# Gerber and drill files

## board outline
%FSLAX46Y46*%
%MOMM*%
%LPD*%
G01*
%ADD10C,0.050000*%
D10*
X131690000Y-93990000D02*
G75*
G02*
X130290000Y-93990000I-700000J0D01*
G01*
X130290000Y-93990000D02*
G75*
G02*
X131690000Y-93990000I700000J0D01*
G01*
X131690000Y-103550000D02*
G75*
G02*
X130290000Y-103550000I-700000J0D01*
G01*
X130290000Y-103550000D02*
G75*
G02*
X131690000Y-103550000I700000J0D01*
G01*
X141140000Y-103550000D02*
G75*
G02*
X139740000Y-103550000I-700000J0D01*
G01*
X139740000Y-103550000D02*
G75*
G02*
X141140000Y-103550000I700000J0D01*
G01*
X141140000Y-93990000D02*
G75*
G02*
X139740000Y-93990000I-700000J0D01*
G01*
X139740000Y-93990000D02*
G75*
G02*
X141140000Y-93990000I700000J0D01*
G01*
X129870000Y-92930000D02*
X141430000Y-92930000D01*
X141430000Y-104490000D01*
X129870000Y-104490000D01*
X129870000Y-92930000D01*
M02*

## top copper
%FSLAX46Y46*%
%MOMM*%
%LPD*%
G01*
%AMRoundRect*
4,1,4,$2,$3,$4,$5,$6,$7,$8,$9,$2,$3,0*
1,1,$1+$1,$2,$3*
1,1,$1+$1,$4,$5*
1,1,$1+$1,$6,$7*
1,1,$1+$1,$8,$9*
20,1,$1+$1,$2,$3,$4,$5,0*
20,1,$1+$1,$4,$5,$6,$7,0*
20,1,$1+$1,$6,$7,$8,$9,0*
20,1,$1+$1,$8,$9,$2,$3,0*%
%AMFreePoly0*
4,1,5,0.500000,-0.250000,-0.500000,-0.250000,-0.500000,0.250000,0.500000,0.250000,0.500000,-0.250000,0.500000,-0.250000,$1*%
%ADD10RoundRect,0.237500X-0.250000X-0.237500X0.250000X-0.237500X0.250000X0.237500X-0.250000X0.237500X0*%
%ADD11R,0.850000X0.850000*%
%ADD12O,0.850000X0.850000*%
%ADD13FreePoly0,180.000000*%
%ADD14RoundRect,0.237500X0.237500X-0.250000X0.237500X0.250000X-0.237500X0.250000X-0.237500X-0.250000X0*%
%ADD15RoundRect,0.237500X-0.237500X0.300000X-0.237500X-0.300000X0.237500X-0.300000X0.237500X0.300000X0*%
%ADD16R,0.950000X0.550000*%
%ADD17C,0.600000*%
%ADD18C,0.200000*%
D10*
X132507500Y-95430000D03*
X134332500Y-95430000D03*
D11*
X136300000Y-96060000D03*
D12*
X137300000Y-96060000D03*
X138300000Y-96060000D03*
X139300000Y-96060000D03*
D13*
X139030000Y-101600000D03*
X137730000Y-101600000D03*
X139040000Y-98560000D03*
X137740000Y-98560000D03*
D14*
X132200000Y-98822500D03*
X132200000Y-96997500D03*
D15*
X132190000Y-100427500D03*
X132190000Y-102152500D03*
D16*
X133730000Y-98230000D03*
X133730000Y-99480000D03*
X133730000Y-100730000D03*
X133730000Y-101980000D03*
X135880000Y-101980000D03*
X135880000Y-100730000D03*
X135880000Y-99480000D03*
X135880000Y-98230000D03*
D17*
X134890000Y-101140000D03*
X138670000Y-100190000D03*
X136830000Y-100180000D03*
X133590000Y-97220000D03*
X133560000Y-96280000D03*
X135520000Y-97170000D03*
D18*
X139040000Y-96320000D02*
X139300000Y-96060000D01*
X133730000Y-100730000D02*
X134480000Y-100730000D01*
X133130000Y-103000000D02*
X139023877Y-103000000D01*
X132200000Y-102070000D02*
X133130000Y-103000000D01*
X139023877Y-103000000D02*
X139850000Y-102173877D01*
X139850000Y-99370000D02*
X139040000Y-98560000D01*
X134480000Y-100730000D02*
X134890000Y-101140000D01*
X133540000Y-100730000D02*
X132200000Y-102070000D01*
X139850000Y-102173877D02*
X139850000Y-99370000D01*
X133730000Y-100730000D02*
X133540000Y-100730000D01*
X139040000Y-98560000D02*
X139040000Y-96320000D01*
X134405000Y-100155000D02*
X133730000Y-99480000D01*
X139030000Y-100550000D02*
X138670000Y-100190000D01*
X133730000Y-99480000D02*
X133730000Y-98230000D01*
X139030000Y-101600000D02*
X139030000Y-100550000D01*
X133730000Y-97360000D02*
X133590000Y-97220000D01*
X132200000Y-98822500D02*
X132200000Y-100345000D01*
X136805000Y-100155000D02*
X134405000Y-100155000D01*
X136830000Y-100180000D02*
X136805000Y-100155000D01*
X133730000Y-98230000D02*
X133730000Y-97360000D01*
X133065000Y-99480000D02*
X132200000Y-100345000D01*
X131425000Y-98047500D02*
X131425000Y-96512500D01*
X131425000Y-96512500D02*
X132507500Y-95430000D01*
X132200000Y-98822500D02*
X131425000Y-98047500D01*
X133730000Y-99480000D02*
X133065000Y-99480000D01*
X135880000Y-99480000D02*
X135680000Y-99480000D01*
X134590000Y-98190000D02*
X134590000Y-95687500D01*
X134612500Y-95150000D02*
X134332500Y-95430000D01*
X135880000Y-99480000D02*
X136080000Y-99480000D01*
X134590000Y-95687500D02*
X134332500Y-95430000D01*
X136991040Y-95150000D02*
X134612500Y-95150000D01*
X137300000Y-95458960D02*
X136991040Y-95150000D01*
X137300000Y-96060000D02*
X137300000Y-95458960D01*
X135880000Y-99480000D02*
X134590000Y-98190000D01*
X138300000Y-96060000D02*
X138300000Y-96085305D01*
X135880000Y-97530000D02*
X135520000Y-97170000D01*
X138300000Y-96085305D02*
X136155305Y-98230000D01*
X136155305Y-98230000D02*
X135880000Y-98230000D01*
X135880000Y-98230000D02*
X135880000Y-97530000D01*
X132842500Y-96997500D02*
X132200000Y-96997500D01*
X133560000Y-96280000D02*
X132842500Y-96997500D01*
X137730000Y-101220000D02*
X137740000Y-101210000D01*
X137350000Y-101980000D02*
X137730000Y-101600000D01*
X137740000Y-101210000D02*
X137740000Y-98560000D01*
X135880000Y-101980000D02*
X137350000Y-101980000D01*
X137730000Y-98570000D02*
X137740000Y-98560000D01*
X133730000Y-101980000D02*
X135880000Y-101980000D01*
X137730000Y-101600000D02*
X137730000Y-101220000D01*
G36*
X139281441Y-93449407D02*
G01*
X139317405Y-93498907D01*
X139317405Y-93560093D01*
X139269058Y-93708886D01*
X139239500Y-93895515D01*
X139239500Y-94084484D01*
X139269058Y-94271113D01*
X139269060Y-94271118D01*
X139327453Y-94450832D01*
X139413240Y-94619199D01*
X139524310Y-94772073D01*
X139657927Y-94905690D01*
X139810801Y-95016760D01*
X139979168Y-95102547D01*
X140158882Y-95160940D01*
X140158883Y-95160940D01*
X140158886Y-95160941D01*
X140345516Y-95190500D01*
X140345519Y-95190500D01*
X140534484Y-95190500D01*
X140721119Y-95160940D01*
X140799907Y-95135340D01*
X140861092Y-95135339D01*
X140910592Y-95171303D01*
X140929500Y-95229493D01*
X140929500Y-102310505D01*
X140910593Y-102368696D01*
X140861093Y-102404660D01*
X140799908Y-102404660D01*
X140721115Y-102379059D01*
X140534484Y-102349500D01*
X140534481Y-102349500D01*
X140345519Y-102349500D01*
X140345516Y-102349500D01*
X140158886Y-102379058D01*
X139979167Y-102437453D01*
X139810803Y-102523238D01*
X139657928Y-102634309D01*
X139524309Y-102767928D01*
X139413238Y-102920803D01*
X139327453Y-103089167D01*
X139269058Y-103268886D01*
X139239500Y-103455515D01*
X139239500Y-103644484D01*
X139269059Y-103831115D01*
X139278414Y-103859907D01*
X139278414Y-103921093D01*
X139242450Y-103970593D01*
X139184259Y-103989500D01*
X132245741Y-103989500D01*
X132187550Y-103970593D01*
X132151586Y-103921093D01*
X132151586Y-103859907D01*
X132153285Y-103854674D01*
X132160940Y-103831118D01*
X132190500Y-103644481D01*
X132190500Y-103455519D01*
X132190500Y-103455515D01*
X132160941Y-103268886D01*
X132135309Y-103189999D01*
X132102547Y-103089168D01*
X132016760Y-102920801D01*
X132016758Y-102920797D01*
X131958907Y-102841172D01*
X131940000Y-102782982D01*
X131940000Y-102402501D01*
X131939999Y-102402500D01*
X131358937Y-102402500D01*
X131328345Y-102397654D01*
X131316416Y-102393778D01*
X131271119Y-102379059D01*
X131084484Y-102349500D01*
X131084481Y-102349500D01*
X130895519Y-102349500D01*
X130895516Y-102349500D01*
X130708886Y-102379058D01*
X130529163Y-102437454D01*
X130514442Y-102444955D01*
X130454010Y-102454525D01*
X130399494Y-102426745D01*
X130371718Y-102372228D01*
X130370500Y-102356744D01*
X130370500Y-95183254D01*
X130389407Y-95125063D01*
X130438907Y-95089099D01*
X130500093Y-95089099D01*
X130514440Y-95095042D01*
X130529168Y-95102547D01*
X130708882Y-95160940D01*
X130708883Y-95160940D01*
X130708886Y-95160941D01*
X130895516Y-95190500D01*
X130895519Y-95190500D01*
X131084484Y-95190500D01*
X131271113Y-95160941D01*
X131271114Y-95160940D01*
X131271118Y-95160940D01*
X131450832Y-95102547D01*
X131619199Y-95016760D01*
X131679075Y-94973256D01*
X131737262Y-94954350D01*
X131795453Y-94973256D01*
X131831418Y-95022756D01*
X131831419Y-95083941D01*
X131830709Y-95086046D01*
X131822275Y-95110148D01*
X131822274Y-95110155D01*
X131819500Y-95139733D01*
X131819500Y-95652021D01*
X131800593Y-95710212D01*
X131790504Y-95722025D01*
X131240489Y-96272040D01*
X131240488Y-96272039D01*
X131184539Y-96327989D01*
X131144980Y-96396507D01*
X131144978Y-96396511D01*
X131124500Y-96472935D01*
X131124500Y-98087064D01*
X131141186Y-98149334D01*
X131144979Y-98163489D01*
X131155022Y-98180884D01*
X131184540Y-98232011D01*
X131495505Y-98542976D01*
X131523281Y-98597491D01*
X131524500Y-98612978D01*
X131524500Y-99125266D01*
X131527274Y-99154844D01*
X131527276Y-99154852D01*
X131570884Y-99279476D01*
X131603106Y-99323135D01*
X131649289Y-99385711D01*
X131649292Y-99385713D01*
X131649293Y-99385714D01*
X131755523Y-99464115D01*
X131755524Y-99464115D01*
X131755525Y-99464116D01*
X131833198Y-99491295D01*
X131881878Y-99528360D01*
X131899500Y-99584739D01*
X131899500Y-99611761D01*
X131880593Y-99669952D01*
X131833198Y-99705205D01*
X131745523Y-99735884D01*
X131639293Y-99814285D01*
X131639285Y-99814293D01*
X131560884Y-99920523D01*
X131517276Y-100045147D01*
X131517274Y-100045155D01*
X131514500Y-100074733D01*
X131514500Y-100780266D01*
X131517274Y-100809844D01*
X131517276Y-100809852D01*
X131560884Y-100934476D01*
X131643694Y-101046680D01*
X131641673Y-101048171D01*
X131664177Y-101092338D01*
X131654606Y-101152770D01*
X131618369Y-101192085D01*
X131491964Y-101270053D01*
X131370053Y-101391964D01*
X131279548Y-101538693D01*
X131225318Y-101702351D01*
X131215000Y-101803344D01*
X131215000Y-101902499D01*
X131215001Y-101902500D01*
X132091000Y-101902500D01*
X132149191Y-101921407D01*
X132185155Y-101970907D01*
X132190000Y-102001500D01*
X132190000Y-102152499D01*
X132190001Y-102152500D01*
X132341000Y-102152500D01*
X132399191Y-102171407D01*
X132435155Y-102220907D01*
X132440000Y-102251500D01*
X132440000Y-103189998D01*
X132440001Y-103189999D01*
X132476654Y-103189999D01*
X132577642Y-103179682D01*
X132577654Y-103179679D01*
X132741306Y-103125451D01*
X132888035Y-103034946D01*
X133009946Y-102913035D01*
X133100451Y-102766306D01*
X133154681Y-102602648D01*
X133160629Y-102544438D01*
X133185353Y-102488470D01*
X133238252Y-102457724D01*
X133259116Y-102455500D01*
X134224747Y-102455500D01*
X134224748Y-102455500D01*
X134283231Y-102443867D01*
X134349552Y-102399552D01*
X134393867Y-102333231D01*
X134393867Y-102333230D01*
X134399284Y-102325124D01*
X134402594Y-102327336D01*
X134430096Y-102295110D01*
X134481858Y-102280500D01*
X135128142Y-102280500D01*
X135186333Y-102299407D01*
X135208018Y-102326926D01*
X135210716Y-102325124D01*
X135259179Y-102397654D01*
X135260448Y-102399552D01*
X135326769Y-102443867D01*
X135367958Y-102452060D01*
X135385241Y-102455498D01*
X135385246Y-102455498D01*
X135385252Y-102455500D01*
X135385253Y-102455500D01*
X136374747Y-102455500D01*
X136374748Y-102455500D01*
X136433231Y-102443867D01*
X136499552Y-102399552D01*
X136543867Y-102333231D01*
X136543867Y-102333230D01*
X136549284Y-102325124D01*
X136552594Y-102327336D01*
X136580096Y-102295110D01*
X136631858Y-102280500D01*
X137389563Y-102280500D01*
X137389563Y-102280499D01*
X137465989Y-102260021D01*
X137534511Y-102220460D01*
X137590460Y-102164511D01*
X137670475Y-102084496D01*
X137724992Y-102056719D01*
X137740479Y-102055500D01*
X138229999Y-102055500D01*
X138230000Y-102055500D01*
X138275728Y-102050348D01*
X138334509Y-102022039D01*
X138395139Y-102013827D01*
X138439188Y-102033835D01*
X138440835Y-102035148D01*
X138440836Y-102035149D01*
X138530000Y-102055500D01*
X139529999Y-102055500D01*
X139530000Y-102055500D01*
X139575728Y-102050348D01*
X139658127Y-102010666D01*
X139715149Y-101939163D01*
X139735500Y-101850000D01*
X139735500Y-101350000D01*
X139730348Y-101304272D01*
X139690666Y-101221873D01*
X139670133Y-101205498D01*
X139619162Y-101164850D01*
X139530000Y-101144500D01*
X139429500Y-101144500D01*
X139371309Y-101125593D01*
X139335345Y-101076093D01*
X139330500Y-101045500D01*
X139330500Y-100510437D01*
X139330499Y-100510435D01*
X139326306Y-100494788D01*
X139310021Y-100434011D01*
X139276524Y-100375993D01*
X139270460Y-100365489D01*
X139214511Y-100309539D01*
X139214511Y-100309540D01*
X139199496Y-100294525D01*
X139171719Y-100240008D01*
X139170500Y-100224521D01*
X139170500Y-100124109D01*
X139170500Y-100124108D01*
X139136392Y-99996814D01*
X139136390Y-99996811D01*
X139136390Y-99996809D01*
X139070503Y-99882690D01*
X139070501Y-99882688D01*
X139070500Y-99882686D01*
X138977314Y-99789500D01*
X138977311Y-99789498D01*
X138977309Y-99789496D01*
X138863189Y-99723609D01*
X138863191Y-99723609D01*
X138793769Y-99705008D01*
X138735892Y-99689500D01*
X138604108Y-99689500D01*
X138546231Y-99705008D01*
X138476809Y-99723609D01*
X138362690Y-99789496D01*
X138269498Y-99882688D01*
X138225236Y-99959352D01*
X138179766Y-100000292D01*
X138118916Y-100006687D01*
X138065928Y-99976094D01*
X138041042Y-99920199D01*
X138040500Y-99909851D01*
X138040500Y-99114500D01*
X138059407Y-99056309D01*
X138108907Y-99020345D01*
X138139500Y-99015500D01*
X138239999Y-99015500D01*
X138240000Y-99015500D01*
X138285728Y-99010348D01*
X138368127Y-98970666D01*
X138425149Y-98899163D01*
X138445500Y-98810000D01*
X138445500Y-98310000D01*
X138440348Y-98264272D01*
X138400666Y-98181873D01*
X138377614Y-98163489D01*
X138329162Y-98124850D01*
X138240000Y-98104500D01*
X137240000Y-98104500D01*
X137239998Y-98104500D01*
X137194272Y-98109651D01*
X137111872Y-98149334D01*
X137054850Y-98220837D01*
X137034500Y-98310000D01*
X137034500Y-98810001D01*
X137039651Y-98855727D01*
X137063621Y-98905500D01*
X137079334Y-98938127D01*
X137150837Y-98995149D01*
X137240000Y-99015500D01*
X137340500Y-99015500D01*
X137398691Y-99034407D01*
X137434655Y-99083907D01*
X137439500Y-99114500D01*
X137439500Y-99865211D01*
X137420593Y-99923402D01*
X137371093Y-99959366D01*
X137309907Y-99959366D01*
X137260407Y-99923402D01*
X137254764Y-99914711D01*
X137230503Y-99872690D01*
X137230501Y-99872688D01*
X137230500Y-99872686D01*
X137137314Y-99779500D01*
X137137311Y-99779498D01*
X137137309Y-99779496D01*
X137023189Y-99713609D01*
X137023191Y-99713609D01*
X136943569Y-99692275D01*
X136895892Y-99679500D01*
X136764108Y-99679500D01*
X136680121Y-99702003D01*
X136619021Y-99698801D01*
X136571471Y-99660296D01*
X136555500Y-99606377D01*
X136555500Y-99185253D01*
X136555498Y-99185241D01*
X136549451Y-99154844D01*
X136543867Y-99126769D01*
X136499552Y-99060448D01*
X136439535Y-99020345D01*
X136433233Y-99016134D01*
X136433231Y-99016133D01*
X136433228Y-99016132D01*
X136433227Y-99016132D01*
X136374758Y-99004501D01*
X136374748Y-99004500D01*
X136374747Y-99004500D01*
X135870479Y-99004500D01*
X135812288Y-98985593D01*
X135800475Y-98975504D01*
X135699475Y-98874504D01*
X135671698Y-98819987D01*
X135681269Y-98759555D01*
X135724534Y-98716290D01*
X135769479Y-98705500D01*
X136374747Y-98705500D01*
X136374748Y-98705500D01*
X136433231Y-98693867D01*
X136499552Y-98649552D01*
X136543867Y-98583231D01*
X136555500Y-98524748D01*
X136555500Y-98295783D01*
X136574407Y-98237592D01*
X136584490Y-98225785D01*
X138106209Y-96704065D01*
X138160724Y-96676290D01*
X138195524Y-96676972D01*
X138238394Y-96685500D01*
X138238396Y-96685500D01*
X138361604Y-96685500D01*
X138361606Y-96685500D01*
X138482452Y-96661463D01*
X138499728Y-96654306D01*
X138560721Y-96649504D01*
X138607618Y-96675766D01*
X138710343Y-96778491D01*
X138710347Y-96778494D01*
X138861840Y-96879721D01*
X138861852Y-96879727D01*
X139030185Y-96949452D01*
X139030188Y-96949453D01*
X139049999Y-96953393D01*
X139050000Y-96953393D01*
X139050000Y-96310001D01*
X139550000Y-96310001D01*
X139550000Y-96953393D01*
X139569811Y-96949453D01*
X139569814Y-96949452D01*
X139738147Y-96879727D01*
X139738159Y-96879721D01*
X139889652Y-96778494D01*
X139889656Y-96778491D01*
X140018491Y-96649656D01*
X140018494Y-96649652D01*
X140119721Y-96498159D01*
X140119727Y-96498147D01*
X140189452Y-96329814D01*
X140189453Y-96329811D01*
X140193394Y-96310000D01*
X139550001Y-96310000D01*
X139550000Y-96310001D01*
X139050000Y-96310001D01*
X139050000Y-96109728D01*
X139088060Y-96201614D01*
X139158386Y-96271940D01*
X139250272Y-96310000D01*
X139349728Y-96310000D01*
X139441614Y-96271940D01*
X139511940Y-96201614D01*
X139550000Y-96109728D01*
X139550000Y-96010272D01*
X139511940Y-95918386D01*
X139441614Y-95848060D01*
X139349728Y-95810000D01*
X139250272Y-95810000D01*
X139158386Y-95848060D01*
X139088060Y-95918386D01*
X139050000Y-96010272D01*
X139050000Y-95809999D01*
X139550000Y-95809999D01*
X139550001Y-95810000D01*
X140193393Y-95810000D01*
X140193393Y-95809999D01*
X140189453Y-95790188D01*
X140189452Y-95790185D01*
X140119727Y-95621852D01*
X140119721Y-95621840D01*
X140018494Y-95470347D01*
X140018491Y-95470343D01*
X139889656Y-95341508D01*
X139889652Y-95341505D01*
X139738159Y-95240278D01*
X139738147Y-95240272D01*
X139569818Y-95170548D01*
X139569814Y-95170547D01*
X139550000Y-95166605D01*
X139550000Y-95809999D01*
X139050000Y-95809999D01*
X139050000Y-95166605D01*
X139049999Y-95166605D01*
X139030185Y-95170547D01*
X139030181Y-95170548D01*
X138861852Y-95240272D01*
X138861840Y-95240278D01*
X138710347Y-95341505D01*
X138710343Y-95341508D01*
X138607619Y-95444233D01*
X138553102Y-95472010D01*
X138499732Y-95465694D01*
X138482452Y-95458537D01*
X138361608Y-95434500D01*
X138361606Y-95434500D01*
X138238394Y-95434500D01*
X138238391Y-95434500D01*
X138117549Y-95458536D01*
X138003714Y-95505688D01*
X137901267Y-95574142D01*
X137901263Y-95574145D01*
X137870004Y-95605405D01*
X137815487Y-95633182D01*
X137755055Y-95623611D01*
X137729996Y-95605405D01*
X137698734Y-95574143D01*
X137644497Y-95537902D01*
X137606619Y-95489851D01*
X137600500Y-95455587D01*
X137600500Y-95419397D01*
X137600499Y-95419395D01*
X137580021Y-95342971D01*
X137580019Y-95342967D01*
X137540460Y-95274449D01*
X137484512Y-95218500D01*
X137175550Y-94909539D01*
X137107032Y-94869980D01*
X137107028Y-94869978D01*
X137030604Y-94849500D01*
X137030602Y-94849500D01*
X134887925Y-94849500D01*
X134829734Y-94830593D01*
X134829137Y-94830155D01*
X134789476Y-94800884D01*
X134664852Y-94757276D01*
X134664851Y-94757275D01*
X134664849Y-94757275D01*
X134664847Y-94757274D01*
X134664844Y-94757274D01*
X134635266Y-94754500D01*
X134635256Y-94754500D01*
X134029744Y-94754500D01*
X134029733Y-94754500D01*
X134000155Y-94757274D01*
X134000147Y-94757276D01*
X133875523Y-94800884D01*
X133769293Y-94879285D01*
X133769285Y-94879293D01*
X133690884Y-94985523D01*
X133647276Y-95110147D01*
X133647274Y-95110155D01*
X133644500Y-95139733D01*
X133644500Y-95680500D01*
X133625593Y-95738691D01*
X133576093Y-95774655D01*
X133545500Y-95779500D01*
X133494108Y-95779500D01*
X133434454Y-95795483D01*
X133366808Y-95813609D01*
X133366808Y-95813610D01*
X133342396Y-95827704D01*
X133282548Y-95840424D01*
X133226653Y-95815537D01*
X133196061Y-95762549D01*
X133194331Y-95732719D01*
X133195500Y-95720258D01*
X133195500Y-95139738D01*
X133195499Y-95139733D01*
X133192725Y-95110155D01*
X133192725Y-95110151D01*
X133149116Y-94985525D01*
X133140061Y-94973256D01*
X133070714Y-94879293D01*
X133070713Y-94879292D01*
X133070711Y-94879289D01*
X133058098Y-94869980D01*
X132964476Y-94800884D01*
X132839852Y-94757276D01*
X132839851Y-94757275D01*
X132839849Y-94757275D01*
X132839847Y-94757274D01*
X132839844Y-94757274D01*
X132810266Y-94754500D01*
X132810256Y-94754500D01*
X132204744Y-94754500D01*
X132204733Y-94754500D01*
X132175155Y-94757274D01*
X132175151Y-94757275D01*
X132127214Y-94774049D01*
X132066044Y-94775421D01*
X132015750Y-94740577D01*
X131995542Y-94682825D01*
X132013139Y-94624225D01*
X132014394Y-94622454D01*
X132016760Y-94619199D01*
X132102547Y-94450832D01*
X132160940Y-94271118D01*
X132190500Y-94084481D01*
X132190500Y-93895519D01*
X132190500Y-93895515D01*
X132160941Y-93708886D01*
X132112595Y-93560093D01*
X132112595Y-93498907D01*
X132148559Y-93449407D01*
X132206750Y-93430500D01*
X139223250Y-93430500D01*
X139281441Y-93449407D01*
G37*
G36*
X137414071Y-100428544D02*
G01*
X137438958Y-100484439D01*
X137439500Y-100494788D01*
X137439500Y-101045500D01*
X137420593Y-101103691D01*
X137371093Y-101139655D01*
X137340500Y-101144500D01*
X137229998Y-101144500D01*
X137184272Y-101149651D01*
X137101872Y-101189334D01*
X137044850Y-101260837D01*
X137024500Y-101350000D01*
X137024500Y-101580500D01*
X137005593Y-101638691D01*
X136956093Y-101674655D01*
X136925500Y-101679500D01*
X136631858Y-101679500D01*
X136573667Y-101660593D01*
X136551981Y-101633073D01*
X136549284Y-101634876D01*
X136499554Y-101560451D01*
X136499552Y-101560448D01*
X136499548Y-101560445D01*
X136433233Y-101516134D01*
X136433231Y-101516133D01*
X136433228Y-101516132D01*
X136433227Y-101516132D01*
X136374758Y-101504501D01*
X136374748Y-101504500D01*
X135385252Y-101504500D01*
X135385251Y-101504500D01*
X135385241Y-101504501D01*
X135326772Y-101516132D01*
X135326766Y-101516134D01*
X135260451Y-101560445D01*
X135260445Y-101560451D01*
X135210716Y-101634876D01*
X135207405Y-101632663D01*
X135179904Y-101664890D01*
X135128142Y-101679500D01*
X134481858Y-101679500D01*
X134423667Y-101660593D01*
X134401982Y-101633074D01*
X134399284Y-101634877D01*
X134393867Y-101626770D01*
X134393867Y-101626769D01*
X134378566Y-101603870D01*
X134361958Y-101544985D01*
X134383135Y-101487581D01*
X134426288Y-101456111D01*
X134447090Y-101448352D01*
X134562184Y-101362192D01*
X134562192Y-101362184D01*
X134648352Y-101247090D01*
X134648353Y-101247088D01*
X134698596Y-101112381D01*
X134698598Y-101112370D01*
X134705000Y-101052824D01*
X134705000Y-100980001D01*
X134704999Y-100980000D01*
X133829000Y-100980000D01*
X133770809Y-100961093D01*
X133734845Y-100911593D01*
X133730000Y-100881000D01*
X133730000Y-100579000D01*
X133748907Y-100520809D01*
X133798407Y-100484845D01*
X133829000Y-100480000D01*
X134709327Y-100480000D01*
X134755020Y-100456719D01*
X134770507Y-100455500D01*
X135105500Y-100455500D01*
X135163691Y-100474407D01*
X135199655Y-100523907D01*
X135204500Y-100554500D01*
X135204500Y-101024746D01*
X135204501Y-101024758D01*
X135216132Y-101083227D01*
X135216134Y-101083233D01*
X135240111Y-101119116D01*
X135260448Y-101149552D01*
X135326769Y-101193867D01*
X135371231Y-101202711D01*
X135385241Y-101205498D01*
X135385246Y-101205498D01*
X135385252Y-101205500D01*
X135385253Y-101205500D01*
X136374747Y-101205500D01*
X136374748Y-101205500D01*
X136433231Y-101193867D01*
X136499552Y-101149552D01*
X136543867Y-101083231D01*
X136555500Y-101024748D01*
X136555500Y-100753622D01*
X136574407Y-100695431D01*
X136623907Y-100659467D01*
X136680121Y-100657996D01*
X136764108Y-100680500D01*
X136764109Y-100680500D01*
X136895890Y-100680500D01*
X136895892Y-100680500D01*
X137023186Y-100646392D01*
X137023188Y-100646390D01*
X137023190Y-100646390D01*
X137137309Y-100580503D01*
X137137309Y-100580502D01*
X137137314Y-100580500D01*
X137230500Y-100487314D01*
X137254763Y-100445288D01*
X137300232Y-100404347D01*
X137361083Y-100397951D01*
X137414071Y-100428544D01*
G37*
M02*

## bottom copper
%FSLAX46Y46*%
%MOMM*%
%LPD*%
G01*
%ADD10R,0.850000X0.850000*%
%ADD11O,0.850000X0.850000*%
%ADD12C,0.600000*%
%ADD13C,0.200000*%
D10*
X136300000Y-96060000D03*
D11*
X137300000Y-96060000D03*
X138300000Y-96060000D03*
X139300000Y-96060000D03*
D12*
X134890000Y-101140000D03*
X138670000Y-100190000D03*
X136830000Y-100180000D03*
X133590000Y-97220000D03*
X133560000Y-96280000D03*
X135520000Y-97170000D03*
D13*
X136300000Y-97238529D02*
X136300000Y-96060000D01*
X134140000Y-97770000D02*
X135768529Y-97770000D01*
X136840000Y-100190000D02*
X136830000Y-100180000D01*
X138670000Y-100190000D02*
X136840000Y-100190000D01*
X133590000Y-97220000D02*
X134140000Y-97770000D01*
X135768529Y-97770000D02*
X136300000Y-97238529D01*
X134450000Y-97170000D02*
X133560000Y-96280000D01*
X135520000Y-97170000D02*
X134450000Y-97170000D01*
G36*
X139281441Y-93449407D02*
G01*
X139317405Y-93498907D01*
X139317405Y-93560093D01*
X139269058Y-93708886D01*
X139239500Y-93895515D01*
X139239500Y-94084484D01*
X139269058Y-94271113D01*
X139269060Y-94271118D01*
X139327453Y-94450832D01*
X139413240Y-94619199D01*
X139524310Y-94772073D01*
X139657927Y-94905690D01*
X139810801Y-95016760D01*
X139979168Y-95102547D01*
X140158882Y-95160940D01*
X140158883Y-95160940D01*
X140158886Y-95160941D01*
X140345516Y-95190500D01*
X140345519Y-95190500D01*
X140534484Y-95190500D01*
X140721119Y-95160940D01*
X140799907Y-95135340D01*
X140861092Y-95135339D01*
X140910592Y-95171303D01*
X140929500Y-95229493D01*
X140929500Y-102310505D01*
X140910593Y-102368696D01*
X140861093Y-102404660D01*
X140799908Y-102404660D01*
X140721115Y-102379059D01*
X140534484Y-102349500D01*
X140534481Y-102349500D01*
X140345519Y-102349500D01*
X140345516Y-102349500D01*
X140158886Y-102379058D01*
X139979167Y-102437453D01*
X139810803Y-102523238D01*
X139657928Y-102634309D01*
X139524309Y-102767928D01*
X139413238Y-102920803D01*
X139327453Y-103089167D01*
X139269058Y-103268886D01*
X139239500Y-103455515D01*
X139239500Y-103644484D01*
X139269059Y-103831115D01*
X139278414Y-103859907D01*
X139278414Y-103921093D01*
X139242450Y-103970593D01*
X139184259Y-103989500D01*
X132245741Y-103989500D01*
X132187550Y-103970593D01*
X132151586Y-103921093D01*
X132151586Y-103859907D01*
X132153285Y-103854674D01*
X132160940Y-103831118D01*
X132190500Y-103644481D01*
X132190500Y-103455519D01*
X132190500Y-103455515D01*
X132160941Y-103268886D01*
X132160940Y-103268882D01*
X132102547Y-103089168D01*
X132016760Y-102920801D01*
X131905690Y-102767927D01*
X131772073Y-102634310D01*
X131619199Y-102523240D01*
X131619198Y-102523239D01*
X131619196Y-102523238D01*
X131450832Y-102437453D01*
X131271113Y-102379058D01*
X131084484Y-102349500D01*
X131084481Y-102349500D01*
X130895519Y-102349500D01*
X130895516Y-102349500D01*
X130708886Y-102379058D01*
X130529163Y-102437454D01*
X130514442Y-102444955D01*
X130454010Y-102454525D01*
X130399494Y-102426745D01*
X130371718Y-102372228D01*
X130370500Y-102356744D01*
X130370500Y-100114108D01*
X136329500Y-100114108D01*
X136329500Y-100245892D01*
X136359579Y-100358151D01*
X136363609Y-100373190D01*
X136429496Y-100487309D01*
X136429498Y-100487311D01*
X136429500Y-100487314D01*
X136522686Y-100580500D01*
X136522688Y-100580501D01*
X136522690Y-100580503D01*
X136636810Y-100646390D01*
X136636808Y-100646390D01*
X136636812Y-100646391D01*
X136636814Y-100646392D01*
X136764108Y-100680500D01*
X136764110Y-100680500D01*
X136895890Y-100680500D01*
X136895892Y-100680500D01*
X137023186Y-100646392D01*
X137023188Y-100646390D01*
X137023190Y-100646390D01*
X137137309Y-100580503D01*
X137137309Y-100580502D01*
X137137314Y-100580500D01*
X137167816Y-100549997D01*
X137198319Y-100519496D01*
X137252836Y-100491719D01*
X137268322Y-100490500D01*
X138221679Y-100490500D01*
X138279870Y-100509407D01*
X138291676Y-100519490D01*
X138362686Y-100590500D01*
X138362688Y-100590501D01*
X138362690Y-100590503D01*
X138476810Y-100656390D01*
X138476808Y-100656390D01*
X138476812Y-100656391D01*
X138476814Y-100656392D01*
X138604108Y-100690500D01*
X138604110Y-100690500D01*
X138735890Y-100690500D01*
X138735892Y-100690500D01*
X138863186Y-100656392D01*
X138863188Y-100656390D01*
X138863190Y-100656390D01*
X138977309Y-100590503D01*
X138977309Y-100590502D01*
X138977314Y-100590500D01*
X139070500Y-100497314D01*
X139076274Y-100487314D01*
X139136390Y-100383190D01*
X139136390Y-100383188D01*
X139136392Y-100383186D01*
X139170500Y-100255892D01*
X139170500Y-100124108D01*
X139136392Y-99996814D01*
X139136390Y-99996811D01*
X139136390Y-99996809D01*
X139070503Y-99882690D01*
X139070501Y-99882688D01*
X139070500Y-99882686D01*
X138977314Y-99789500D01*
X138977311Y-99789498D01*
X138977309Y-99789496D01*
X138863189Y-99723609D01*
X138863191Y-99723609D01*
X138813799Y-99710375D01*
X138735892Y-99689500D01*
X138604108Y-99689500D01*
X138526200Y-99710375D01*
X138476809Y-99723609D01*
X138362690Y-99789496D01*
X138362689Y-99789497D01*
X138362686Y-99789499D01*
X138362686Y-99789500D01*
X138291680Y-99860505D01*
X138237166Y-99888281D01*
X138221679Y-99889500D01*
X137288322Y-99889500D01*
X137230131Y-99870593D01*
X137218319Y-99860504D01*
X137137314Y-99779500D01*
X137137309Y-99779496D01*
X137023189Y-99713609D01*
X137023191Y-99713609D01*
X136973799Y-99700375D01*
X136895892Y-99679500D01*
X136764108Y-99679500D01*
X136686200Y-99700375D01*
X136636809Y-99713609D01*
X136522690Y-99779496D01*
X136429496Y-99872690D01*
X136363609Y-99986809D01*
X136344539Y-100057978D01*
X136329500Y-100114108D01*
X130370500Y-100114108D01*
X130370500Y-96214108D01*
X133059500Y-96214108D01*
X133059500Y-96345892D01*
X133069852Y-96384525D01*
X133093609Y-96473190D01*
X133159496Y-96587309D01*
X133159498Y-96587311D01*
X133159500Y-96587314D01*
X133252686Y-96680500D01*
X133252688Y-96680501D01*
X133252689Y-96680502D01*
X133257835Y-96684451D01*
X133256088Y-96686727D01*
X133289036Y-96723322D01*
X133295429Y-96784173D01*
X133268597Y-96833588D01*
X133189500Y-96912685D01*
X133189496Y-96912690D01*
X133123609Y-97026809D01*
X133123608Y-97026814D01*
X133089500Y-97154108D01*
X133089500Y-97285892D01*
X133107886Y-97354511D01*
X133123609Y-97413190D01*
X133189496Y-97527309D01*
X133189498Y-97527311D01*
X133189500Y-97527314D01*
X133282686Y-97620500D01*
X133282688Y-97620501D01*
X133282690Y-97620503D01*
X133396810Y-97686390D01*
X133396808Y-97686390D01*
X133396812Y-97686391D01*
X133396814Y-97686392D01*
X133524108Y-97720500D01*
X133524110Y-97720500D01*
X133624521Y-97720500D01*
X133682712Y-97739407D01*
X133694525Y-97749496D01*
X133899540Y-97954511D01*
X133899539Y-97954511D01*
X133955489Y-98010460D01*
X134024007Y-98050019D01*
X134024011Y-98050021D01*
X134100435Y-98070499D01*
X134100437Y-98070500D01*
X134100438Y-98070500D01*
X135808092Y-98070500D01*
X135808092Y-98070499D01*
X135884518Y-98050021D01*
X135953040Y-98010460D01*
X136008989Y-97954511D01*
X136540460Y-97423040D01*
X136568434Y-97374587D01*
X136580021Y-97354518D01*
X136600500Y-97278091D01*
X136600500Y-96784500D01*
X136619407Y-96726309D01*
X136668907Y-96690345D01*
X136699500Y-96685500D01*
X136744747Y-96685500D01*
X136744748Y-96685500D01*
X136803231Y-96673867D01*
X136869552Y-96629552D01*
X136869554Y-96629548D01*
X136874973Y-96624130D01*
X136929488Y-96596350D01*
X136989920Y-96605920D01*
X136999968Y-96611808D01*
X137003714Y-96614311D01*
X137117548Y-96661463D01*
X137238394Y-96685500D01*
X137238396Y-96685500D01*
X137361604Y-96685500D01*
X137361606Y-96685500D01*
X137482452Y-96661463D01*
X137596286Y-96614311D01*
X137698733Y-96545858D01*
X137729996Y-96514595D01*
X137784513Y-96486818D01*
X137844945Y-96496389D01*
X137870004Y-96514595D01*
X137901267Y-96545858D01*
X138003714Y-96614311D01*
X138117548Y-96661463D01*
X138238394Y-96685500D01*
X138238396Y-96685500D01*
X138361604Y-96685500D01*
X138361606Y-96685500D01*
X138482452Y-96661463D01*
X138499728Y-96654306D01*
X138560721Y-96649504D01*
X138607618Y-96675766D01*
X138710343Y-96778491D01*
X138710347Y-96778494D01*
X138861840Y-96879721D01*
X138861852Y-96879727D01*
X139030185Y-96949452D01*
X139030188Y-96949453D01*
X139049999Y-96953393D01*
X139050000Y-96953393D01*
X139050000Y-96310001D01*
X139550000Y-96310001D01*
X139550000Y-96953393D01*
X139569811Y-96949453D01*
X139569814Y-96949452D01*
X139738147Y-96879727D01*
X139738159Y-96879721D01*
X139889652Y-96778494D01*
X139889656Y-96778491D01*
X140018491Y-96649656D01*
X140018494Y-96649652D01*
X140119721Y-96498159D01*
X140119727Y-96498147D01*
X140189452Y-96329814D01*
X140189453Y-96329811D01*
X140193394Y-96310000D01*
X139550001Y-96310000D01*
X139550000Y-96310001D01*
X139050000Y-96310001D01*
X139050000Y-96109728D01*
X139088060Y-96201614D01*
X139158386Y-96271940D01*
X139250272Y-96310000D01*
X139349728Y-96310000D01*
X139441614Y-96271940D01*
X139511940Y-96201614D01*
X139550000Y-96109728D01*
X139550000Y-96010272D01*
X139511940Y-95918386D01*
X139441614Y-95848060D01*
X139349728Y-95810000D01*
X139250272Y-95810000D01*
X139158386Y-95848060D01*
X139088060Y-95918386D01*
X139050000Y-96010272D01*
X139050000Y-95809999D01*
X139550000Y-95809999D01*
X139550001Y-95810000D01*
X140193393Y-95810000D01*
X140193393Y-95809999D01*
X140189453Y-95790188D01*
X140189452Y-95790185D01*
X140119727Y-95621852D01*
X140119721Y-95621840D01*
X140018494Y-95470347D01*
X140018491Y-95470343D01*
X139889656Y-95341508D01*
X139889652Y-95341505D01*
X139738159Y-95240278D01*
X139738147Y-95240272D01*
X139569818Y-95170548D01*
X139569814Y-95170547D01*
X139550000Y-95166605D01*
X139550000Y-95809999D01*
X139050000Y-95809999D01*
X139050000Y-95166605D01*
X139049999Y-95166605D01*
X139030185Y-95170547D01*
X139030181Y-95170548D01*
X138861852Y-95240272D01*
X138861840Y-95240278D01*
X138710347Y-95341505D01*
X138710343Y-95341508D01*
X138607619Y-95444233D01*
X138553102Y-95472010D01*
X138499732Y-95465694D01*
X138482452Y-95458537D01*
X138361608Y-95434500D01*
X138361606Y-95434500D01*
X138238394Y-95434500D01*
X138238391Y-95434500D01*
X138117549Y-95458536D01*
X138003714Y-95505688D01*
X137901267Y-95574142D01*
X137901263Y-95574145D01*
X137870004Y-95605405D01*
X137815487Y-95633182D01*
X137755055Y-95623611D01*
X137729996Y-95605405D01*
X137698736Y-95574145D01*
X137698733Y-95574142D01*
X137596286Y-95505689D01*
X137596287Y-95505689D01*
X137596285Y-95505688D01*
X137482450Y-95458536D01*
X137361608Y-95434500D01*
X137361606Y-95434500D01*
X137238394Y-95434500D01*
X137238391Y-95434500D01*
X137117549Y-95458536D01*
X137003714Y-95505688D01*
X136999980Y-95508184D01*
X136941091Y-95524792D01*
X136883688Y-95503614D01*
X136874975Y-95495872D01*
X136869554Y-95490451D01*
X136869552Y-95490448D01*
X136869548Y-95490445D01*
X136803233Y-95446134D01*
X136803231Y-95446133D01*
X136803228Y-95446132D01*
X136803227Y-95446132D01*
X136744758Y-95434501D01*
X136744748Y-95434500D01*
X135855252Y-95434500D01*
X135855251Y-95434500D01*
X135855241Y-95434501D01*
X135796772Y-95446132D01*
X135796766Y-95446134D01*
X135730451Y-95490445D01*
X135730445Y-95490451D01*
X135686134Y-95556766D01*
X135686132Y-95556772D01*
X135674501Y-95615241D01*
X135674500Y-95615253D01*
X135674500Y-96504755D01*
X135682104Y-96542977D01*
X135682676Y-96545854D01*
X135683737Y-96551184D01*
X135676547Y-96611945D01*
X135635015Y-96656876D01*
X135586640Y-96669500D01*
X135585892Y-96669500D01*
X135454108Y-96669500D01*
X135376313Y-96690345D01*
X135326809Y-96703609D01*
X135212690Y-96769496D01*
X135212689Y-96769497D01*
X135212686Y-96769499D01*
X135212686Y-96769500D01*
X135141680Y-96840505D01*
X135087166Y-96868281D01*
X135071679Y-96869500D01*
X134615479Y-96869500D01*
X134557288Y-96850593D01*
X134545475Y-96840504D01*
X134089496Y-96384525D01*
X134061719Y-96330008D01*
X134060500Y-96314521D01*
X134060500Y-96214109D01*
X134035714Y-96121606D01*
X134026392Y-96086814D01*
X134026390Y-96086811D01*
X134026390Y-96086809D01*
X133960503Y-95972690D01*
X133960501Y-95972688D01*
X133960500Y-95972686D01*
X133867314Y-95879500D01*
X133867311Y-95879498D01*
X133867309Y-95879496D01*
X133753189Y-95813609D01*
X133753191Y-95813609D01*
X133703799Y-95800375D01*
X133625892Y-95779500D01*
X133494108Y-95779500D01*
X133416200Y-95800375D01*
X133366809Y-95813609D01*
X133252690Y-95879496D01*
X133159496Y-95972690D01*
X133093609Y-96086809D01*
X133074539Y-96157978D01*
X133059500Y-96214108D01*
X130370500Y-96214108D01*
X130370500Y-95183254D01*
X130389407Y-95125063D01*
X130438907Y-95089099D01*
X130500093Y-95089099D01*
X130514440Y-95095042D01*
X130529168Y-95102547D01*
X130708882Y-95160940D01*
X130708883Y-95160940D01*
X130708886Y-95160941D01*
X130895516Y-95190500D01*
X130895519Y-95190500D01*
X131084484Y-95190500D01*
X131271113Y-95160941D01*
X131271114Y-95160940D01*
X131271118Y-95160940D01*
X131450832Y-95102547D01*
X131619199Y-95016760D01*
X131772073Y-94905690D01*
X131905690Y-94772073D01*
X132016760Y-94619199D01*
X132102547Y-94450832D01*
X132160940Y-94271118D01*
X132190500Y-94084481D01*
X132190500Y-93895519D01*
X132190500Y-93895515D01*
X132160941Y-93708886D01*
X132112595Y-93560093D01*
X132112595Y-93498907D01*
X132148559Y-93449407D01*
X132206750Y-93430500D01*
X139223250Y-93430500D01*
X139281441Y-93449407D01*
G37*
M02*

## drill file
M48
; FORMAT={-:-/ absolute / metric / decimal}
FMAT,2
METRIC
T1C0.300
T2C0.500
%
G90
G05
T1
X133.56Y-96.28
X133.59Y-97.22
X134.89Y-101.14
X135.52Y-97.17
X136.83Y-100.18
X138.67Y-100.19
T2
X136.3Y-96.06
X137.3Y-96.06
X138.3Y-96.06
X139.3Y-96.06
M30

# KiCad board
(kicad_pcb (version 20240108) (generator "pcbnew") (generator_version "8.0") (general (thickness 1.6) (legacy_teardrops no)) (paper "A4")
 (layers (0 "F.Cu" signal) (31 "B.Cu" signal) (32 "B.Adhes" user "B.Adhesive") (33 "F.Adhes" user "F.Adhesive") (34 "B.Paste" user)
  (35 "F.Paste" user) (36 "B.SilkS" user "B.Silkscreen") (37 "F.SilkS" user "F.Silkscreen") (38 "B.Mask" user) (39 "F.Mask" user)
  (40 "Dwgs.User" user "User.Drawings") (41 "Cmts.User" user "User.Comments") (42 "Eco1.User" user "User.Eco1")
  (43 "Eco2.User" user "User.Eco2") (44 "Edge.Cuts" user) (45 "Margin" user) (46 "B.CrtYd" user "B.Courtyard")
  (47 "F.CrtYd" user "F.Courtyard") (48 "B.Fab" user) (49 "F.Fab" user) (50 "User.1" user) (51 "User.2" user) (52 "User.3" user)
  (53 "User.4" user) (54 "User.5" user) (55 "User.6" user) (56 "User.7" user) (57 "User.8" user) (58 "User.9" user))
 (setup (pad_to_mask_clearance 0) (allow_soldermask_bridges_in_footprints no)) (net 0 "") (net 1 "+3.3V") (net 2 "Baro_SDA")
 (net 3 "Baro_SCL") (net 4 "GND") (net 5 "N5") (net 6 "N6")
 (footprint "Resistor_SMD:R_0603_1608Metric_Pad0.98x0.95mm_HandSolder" (layer "F.Cu") (at 133.42 95.43)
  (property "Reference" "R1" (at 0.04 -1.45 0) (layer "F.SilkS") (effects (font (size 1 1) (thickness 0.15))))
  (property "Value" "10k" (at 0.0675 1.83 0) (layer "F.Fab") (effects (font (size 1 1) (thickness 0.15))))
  (pad "1" smd roundrect (at -0.9125 0) (size 0.975 0.95) (layers "F.Cu" "F.Paste" "F.Mask") (roundrect_rratio 0.25) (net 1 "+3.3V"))
  (pad "2" smd roundrect (at 0.9125 0) (size 0.975 0.95) (layers "F.Cu" "F.Paste" "F.Mask") (roundrect_rratio 0.25) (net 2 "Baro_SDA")))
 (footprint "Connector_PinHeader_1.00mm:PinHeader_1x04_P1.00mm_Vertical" (layer "F.Cu") (at 136.3 96.06 90)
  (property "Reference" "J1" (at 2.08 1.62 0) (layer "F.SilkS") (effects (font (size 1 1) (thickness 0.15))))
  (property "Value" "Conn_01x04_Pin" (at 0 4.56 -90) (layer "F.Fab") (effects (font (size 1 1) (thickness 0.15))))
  (pad "1" thru_hole rect (at 0 0 90) (size 0.85 0.85) (drill 0.5) (layers "*.Cu" "*.Mask") (remove_unused_layers no) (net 1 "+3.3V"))
  (pad "2" thru_hole oval (at 0 1 90) (size 0.85 0.85) (drill 0.5) (layers "*.Cu" "*.Mask") (remove_unused_layers no) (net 2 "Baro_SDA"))
  (pad "3" thru_hole oval (at 0 2 90) (size 0.85 0.85) (drill 0.5) (layers "*.Cu" "*.Mask") (remove_unused_layers no) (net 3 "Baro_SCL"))
  (pad "4" thru_hole oval (at 0 3 90) (size 0.85 0.85) (drill 0.5) (layers "*.Cu" "*.Mask") (remove_unused_layers no) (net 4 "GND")))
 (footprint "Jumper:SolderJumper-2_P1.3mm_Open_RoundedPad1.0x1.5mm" (layer "F.Cu") (at 138.38 101.6 180)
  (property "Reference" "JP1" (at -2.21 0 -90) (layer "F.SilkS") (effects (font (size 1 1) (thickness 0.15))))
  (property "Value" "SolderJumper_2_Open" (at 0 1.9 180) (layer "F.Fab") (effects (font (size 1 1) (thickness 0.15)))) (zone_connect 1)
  (pad "1" smd custom (at -0.65 0 180) (size 1 0.5) (layers "F.Cu" "F.Mask") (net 1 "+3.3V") (zone_connect 2) (thermal_bridge_angle 45)
   (options (clearance outline) (anchor rect)) (primitives))
  (pad "2" smd custom (at 0.65 0 180) (size 1 0.5) (layers "F.Cu" "F.Mask") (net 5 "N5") (zone_connect 2) (thermal_bridge_angle 45)
   (options (clearance outline) (anchor rect)) (primitives)))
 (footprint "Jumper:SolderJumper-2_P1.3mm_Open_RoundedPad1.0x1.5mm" (layer "F.Cu") (at 138.39 98.56 180)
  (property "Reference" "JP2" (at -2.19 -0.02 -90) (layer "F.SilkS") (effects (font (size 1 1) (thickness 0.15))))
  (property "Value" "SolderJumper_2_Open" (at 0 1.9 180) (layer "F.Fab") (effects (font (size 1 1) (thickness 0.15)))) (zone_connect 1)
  (pad "1" smd custom (at -0.65 0 180) (size 1 0.5) (layers "F.Cu" "F.Mask") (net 4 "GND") (zone_connect 2) (thermal_bridge_angle 45)
   (options (clearance outline) (anchor rect)) (primitives))
  (pad "2" smd custom (at 0.65 0 180) (size 1 0.5) (layers "F.Cu" "F.Mask") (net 5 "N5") (zone_connect 2) (thermal_bridge_angle 45)
   (options (clearance outline) (anchor rect)) (primitives)))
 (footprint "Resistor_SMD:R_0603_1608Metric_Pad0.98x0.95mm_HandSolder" (layer "F.Cu") (at 132.2 97.91 90)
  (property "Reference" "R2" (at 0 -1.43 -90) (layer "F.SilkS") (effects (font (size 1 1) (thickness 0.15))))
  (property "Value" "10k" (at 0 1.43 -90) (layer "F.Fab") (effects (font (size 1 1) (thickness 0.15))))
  (pad "1" smd roundrect (at -0.9125 0 90) (size 0.975 0.95) (layers "F.Cu" "F.Paste" "F.Mask") (roundrect_rratio 0.25) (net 1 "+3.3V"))
  (pad "2" smd roundrect (at 0.9125 0 90) (size 0.975 0.95) (layers "F.Cu" "F.Paste" "F.Mask") (roundrect_rratio 0.25) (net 3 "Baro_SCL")))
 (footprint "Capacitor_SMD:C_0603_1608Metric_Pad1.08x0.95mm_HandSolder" (layer "F.Cu") (at 132.19 101.29 -90)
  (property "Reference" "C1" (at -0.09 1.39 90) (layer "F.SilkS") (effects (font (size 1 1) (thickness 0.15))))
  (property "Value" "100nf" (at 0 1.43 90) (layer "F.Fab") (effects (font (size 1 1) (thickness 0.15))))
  (pad "1" smd roundrect (at -0.8625 0 270) (size 1.075 0.95) (layers "F.Cu" "F.Paste" "F.Mask") (roundrect_rratio 0.25) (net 1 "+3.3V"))
  (pad "2" smd roundrect (at 0.8625 0 270) (size 1.075 0.95) (layers "F.Cu" "F.Paste" "F.Mask") (roundrect_rratio 0.25) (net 4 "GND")))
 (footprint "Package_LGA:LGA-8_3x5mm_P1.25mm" (layer "F.Cu") (at 134.805 100.105)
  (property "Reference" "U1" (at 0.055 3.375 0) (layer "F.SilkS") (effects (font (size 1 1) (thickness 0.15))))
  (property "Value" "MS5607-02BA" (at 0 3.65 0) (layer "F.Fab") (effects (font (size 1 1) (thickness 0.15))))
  (pad "1" smd rect (at -1.075 -1.875) (size 0.95 0.55) (layers "F.Cu" "F.Paste" "F.Mask") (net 1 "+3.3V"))
  (pad "2" smd rect (at -1.075 -0.625) (size 0.95 0.55) (layers "F.Cu" "F.Paste" "F.Mask") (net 1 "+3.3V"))
  (pad "3" smd rect (at -1.075 0.625) (size 0.95 0.55) (layers "F.Cu" "F.Paste" "F.Mask") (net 4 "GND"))
  (pad "4" smd rect (at -1.075 1.875) (size 0.95 0.55) (layers "F.Cu" "F.Paste" "F.Mask") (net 5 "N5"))
  (pad "5" smd rect (at 1.075 1.875) (size 0.95 0.55) (layers "F.Cu" "F.Paste" "F.Mask") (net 5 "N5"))
  (pad "6" smd rect (at 1.075 0.625) (size 0.95 0.55) (layers "F.Cu" "F.Paste" "F.Mask") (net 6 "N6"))
  (pad "7" smd rect (at 1.075 -0.625) (size 0.95 0.55) (layers "F.Cu" "F.Paste" "F.Mask") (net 2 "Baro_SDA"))
  (pad "8" smd rect (at 1.075 -1.875) (size 0.95 0.55) (layers "F.Cu" "F.Paste" "F.Mask") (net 3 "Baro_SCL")))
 (gr_circle (center 130.99 93.99) (end 131.69 93.99) (stroke (width 0.05) (type default)) (fill none) (layer "Edge.Cuts"))
 (gr_circle (center 130.99 103.55) (end 131.69 103.55) (stroke (width 0.05) (type default)) (fill none) (layer "Edge.Cuts"))
 (gr_circle (center 140.44 103.55) (end 141.14 103.55) (stroke (width 0.05) (type default)) (fill none) (layer "Edge.Cuts"))
 (gr_circle (center 140.44 93.99) (end 141.14 93.99) (stroke (width 0.05) (type default)) (fill none) (layer "Edge.Cuts"))
 (gr_rect (start 129.87 92.93) (end 141.43 104.49) (stroke (width 0.05) (type default)) (fill none) (layer "Edge.Cuts"))
 (segment (start 139.04 96.32) (end 139.3 96.06) (width 0.2) (layer "F.Cu") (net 4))
 (segment (start 133.73 100.73) (end 134.48 100.73) (width 0.2) (layer "F.Cu") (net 4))
 (segment (start 133.13 103) (end 139.023877 103) (width 0.2) (layer "F.Cu") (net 4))
 (segment (start 132.2 102.07) (end 133.13 103) (width 0.2) (layer "F.Cu") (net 4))
 (segment (start 139.023877 103) (end 139.85 102.173877) (width 0.2) (layer "F.Cu") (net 4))
 (segment (start 139.85 99.37) (end 139.04 98.56) (width 0.2) (layer "F.Cu") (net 4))
 (segment (start 134.48 100.73) (end 134.89 101.14) (width 0.2) (layer "F.Cu") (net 4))
 (segment (start 133.54 100.73) (end 132.2 102.07) (width 0.2) (layer "F.Cu") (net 4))
 (segment (start 139.85 102.173877) (end 139.85 99.37) (width 0.2) (layer "F.Cu") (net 4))
 (segment (start 133.73 100.73) (end 133.54 100.73) (width 0.2) (layer "F.Cu") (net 4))
 (segment (start 139.04 98.56) (end 139.04 96.32) (width 0.2) (layer "F.Cu") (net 4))
 (via (at 134.89 101.14) (size 0.6) (drill 0.3) (layers "F.Cu" "B.Cu") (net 4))
 (segment (start 134.405 100.155) (end 133.73 99.48) (width 0.2) (layer "F.Cu") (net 1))
 (segment (start 139.03 100.55) (end 138.67 100.19) (width 0.2) (layer "F.Cu") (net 1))
 (segment (start 133.73 99.48) (end 133.73 98.23) (width 0.2) (layer "F.Cu") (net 1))
 (segment (start 139.03 101.6) (end 139.03 100.55) (width 0.2) (layer "F.Cu") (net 1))
 (segment (start 133.73 97.36) (end 133.59 97.22) (width 0.2) (layer "F.Cu") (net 1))
 (segment (start 132.2 98.8225) (end 132.2 100.345) (width 0.2) (layer "F.Cu") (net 1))
 (segment (start 136.805 100.155) (end 134.405 100.155) (width 0.2) (layer "F.Cu") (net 1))
 (segment (start 136.83 100.18) (end 136.805 100.155) (width 0.2) (layer "F.Cu") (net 1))
 (segment (start 133.73 98.23) (end 133.73 97.36) (width 0.2) (layer "F.Cu") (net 1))
 (segment (start 133.065 99.48) (end 132.2 100.345) (width 0.2) (layer "F.Cu") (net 1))
 (segment (start 131.425 98.0475) (end 131.425 96.5125) (width 0.2) (layer "F.Cu") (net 1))
 (segment (start 131.425 96.5125) (end 132.5075 95.43) (width 0.2) (layer "F.Cu") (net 1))
 (segment (start 132.2 98.8225) (end 131.425 98.0475) (width 0.2) (layer "F.Cu") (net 1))
 (segment (start 133.73 99.48) (end 133.065 99.48) (width 0.2) (layer "F.Cu") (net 1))
 (via (at 138.67 100.19) (size 0.6) (drill 0.3) (layers "F.Cu" "B.Cu") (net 1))
 (via (at 136.83 100.18) (size 0.6) (drill 0.3) (layers "F.Cu" "B.Cu") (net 1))
 (via (at 133.59 97.22) (size 0.6) (drill 0.3) (layers "F.Cu" "B.Cu") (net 1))
 (segment (start 136.3 97.238529) (end 136.3 96.06) (width 0.2) (layer "B.Cu") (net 1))
 (segment (start 134.14 97.77) (end 135.768529 97.77) (width 0.2) (layer "B.Cu") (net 1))
 (segment (start 136.84 100.19) (end 136.83 100.18) (width 0.2) (layer "B.Cu") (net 1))
 (segment (start 138.67 100.19) (end 136.84 100.19) (width 0.2) (layer "B.Cu") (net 1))
 (segment (start 133.59 97.22) (end 134.14 97.77) (width 0.2) (layer "B.Cu") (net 1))
 (segment (start 135.768529 97.77) (end 136.3 97.238529) (width 0.2) (layer "B.Cu") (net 1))
 (segment (start 135.88 99.48) (end 135.68 99.48) (width 0.2) (layer "F.Cu") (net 2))
 (segment (start 134.59 98.19) (end 134.59 95.6875) (width 0.2) (layer "F.Cu") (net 2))
 (segment (start 134.6125 95.15) (end 134.3325 95.43) (width 0.2) (layer "F.Cu") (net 2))
 (segment (start 135.88 99.48) (end 136.08 99.48) (width 0.2) (layer "F.Cu") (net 2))
 (segment (start 134.59 95.6875) (end 134.3325 95.43) (width 0.2) (layer "F.Cu") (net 2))
 (segment (start 136.99104 95.15) (end 134.6125 95.15) (width 0.2) (layer "F.Cu") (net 2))
 (segment (start 137.3 95.45896) (end 136.99104 95.15) (width 0.2) (layer "F.Cu") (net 2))
 (segment (start 137.3 96.06) (end 137.3 95.45896) (width 0.2) (layer "F.Cu") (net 2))
 (segment (start 135.88 99.48) (end 134.59 98.19) (width 0.2) (layer "F.Cu") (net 2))
 (segment (start 138.3 96.06) (end 138.3 96.085305) (width 0.2) (layer "F.Cu") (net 3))
 (segment (start 135.88 97.53) (end 135.52 97.17) (width 0.2) (layer "F.Cu") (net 3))
 (segment (start 138.3 96.085305) (end 136.155305 98.23) (width 0.2) (layer "F.Cu") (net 3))
 (segment (start 136.155305 98.23) (end 135.88 98.23) (width 0.2) (layer "F.Cu") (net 3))
 (segment (start 135.88 98.23) (end 135.88 97.53) (width 0.2) (layer "F.Cu") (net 3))
 (segment (start 132.8425 96.9975) (end 132.2 96.9975) (width 0.2) (layer "F.Cu") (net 3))
 (segment (start 133.56 96.28) (end 132.8425 96.9975) (width 0.2) (layer "F.Cu") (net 3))
 (via (at 133.56 96.28) (size 0.6) (drill 0.3) (layers "F.Cu" "B.Cu") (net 3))
 (via (at 135.52 97.17) (size 0.6) (drill 0.3) (layers "F.Cu" "B.Cu") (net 3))
 (segment (start 134.45 97.17) (end 133.56 96.28) (width 0.2) (layer "B.Cu") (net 3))
 (segment (start 135.52 97.17) (end 134.45 97.17) (width 0.2) (layer "B.Cu") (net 3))
 (segment (start 137.73 101.22) (end 137.74 101.21) (width 0.2) (layer "F.Cu") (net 5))
 (segment (start 137.35 101.98) (end 137.73 101.6) (width 0.2) (layer "F.Cu") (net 5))
 (segment (start 137.74 101.21) (end 137.74 98.56) (width 0.2) (layer "F.Cu") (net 5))
 (segment (start 135.88 101.98) (end 137.35 101.98) (width 0.2) (layer "F.Cu") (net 5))
 (segment (start 137.73 98.57) (end 137.74 98.56) (width 0.2) (layer "F.Cu") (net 5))
 (segment (start 133.73 101.98) (end 135.88 101.98) (width 0.2) (layer "F.Cu") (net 5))
 (segment (start 137.73 101.6) (end 137.73 101.22) (width 0.2) (layer "F.Cu") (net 5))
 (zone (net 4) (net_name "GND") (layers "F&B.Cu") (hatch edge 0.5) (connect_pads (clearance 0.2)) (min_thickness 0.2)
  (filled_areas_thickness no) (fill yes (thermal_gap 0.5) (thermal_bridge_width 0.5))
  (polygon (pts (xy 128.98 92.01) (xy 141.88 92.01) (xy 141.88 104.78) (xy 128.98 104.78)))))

